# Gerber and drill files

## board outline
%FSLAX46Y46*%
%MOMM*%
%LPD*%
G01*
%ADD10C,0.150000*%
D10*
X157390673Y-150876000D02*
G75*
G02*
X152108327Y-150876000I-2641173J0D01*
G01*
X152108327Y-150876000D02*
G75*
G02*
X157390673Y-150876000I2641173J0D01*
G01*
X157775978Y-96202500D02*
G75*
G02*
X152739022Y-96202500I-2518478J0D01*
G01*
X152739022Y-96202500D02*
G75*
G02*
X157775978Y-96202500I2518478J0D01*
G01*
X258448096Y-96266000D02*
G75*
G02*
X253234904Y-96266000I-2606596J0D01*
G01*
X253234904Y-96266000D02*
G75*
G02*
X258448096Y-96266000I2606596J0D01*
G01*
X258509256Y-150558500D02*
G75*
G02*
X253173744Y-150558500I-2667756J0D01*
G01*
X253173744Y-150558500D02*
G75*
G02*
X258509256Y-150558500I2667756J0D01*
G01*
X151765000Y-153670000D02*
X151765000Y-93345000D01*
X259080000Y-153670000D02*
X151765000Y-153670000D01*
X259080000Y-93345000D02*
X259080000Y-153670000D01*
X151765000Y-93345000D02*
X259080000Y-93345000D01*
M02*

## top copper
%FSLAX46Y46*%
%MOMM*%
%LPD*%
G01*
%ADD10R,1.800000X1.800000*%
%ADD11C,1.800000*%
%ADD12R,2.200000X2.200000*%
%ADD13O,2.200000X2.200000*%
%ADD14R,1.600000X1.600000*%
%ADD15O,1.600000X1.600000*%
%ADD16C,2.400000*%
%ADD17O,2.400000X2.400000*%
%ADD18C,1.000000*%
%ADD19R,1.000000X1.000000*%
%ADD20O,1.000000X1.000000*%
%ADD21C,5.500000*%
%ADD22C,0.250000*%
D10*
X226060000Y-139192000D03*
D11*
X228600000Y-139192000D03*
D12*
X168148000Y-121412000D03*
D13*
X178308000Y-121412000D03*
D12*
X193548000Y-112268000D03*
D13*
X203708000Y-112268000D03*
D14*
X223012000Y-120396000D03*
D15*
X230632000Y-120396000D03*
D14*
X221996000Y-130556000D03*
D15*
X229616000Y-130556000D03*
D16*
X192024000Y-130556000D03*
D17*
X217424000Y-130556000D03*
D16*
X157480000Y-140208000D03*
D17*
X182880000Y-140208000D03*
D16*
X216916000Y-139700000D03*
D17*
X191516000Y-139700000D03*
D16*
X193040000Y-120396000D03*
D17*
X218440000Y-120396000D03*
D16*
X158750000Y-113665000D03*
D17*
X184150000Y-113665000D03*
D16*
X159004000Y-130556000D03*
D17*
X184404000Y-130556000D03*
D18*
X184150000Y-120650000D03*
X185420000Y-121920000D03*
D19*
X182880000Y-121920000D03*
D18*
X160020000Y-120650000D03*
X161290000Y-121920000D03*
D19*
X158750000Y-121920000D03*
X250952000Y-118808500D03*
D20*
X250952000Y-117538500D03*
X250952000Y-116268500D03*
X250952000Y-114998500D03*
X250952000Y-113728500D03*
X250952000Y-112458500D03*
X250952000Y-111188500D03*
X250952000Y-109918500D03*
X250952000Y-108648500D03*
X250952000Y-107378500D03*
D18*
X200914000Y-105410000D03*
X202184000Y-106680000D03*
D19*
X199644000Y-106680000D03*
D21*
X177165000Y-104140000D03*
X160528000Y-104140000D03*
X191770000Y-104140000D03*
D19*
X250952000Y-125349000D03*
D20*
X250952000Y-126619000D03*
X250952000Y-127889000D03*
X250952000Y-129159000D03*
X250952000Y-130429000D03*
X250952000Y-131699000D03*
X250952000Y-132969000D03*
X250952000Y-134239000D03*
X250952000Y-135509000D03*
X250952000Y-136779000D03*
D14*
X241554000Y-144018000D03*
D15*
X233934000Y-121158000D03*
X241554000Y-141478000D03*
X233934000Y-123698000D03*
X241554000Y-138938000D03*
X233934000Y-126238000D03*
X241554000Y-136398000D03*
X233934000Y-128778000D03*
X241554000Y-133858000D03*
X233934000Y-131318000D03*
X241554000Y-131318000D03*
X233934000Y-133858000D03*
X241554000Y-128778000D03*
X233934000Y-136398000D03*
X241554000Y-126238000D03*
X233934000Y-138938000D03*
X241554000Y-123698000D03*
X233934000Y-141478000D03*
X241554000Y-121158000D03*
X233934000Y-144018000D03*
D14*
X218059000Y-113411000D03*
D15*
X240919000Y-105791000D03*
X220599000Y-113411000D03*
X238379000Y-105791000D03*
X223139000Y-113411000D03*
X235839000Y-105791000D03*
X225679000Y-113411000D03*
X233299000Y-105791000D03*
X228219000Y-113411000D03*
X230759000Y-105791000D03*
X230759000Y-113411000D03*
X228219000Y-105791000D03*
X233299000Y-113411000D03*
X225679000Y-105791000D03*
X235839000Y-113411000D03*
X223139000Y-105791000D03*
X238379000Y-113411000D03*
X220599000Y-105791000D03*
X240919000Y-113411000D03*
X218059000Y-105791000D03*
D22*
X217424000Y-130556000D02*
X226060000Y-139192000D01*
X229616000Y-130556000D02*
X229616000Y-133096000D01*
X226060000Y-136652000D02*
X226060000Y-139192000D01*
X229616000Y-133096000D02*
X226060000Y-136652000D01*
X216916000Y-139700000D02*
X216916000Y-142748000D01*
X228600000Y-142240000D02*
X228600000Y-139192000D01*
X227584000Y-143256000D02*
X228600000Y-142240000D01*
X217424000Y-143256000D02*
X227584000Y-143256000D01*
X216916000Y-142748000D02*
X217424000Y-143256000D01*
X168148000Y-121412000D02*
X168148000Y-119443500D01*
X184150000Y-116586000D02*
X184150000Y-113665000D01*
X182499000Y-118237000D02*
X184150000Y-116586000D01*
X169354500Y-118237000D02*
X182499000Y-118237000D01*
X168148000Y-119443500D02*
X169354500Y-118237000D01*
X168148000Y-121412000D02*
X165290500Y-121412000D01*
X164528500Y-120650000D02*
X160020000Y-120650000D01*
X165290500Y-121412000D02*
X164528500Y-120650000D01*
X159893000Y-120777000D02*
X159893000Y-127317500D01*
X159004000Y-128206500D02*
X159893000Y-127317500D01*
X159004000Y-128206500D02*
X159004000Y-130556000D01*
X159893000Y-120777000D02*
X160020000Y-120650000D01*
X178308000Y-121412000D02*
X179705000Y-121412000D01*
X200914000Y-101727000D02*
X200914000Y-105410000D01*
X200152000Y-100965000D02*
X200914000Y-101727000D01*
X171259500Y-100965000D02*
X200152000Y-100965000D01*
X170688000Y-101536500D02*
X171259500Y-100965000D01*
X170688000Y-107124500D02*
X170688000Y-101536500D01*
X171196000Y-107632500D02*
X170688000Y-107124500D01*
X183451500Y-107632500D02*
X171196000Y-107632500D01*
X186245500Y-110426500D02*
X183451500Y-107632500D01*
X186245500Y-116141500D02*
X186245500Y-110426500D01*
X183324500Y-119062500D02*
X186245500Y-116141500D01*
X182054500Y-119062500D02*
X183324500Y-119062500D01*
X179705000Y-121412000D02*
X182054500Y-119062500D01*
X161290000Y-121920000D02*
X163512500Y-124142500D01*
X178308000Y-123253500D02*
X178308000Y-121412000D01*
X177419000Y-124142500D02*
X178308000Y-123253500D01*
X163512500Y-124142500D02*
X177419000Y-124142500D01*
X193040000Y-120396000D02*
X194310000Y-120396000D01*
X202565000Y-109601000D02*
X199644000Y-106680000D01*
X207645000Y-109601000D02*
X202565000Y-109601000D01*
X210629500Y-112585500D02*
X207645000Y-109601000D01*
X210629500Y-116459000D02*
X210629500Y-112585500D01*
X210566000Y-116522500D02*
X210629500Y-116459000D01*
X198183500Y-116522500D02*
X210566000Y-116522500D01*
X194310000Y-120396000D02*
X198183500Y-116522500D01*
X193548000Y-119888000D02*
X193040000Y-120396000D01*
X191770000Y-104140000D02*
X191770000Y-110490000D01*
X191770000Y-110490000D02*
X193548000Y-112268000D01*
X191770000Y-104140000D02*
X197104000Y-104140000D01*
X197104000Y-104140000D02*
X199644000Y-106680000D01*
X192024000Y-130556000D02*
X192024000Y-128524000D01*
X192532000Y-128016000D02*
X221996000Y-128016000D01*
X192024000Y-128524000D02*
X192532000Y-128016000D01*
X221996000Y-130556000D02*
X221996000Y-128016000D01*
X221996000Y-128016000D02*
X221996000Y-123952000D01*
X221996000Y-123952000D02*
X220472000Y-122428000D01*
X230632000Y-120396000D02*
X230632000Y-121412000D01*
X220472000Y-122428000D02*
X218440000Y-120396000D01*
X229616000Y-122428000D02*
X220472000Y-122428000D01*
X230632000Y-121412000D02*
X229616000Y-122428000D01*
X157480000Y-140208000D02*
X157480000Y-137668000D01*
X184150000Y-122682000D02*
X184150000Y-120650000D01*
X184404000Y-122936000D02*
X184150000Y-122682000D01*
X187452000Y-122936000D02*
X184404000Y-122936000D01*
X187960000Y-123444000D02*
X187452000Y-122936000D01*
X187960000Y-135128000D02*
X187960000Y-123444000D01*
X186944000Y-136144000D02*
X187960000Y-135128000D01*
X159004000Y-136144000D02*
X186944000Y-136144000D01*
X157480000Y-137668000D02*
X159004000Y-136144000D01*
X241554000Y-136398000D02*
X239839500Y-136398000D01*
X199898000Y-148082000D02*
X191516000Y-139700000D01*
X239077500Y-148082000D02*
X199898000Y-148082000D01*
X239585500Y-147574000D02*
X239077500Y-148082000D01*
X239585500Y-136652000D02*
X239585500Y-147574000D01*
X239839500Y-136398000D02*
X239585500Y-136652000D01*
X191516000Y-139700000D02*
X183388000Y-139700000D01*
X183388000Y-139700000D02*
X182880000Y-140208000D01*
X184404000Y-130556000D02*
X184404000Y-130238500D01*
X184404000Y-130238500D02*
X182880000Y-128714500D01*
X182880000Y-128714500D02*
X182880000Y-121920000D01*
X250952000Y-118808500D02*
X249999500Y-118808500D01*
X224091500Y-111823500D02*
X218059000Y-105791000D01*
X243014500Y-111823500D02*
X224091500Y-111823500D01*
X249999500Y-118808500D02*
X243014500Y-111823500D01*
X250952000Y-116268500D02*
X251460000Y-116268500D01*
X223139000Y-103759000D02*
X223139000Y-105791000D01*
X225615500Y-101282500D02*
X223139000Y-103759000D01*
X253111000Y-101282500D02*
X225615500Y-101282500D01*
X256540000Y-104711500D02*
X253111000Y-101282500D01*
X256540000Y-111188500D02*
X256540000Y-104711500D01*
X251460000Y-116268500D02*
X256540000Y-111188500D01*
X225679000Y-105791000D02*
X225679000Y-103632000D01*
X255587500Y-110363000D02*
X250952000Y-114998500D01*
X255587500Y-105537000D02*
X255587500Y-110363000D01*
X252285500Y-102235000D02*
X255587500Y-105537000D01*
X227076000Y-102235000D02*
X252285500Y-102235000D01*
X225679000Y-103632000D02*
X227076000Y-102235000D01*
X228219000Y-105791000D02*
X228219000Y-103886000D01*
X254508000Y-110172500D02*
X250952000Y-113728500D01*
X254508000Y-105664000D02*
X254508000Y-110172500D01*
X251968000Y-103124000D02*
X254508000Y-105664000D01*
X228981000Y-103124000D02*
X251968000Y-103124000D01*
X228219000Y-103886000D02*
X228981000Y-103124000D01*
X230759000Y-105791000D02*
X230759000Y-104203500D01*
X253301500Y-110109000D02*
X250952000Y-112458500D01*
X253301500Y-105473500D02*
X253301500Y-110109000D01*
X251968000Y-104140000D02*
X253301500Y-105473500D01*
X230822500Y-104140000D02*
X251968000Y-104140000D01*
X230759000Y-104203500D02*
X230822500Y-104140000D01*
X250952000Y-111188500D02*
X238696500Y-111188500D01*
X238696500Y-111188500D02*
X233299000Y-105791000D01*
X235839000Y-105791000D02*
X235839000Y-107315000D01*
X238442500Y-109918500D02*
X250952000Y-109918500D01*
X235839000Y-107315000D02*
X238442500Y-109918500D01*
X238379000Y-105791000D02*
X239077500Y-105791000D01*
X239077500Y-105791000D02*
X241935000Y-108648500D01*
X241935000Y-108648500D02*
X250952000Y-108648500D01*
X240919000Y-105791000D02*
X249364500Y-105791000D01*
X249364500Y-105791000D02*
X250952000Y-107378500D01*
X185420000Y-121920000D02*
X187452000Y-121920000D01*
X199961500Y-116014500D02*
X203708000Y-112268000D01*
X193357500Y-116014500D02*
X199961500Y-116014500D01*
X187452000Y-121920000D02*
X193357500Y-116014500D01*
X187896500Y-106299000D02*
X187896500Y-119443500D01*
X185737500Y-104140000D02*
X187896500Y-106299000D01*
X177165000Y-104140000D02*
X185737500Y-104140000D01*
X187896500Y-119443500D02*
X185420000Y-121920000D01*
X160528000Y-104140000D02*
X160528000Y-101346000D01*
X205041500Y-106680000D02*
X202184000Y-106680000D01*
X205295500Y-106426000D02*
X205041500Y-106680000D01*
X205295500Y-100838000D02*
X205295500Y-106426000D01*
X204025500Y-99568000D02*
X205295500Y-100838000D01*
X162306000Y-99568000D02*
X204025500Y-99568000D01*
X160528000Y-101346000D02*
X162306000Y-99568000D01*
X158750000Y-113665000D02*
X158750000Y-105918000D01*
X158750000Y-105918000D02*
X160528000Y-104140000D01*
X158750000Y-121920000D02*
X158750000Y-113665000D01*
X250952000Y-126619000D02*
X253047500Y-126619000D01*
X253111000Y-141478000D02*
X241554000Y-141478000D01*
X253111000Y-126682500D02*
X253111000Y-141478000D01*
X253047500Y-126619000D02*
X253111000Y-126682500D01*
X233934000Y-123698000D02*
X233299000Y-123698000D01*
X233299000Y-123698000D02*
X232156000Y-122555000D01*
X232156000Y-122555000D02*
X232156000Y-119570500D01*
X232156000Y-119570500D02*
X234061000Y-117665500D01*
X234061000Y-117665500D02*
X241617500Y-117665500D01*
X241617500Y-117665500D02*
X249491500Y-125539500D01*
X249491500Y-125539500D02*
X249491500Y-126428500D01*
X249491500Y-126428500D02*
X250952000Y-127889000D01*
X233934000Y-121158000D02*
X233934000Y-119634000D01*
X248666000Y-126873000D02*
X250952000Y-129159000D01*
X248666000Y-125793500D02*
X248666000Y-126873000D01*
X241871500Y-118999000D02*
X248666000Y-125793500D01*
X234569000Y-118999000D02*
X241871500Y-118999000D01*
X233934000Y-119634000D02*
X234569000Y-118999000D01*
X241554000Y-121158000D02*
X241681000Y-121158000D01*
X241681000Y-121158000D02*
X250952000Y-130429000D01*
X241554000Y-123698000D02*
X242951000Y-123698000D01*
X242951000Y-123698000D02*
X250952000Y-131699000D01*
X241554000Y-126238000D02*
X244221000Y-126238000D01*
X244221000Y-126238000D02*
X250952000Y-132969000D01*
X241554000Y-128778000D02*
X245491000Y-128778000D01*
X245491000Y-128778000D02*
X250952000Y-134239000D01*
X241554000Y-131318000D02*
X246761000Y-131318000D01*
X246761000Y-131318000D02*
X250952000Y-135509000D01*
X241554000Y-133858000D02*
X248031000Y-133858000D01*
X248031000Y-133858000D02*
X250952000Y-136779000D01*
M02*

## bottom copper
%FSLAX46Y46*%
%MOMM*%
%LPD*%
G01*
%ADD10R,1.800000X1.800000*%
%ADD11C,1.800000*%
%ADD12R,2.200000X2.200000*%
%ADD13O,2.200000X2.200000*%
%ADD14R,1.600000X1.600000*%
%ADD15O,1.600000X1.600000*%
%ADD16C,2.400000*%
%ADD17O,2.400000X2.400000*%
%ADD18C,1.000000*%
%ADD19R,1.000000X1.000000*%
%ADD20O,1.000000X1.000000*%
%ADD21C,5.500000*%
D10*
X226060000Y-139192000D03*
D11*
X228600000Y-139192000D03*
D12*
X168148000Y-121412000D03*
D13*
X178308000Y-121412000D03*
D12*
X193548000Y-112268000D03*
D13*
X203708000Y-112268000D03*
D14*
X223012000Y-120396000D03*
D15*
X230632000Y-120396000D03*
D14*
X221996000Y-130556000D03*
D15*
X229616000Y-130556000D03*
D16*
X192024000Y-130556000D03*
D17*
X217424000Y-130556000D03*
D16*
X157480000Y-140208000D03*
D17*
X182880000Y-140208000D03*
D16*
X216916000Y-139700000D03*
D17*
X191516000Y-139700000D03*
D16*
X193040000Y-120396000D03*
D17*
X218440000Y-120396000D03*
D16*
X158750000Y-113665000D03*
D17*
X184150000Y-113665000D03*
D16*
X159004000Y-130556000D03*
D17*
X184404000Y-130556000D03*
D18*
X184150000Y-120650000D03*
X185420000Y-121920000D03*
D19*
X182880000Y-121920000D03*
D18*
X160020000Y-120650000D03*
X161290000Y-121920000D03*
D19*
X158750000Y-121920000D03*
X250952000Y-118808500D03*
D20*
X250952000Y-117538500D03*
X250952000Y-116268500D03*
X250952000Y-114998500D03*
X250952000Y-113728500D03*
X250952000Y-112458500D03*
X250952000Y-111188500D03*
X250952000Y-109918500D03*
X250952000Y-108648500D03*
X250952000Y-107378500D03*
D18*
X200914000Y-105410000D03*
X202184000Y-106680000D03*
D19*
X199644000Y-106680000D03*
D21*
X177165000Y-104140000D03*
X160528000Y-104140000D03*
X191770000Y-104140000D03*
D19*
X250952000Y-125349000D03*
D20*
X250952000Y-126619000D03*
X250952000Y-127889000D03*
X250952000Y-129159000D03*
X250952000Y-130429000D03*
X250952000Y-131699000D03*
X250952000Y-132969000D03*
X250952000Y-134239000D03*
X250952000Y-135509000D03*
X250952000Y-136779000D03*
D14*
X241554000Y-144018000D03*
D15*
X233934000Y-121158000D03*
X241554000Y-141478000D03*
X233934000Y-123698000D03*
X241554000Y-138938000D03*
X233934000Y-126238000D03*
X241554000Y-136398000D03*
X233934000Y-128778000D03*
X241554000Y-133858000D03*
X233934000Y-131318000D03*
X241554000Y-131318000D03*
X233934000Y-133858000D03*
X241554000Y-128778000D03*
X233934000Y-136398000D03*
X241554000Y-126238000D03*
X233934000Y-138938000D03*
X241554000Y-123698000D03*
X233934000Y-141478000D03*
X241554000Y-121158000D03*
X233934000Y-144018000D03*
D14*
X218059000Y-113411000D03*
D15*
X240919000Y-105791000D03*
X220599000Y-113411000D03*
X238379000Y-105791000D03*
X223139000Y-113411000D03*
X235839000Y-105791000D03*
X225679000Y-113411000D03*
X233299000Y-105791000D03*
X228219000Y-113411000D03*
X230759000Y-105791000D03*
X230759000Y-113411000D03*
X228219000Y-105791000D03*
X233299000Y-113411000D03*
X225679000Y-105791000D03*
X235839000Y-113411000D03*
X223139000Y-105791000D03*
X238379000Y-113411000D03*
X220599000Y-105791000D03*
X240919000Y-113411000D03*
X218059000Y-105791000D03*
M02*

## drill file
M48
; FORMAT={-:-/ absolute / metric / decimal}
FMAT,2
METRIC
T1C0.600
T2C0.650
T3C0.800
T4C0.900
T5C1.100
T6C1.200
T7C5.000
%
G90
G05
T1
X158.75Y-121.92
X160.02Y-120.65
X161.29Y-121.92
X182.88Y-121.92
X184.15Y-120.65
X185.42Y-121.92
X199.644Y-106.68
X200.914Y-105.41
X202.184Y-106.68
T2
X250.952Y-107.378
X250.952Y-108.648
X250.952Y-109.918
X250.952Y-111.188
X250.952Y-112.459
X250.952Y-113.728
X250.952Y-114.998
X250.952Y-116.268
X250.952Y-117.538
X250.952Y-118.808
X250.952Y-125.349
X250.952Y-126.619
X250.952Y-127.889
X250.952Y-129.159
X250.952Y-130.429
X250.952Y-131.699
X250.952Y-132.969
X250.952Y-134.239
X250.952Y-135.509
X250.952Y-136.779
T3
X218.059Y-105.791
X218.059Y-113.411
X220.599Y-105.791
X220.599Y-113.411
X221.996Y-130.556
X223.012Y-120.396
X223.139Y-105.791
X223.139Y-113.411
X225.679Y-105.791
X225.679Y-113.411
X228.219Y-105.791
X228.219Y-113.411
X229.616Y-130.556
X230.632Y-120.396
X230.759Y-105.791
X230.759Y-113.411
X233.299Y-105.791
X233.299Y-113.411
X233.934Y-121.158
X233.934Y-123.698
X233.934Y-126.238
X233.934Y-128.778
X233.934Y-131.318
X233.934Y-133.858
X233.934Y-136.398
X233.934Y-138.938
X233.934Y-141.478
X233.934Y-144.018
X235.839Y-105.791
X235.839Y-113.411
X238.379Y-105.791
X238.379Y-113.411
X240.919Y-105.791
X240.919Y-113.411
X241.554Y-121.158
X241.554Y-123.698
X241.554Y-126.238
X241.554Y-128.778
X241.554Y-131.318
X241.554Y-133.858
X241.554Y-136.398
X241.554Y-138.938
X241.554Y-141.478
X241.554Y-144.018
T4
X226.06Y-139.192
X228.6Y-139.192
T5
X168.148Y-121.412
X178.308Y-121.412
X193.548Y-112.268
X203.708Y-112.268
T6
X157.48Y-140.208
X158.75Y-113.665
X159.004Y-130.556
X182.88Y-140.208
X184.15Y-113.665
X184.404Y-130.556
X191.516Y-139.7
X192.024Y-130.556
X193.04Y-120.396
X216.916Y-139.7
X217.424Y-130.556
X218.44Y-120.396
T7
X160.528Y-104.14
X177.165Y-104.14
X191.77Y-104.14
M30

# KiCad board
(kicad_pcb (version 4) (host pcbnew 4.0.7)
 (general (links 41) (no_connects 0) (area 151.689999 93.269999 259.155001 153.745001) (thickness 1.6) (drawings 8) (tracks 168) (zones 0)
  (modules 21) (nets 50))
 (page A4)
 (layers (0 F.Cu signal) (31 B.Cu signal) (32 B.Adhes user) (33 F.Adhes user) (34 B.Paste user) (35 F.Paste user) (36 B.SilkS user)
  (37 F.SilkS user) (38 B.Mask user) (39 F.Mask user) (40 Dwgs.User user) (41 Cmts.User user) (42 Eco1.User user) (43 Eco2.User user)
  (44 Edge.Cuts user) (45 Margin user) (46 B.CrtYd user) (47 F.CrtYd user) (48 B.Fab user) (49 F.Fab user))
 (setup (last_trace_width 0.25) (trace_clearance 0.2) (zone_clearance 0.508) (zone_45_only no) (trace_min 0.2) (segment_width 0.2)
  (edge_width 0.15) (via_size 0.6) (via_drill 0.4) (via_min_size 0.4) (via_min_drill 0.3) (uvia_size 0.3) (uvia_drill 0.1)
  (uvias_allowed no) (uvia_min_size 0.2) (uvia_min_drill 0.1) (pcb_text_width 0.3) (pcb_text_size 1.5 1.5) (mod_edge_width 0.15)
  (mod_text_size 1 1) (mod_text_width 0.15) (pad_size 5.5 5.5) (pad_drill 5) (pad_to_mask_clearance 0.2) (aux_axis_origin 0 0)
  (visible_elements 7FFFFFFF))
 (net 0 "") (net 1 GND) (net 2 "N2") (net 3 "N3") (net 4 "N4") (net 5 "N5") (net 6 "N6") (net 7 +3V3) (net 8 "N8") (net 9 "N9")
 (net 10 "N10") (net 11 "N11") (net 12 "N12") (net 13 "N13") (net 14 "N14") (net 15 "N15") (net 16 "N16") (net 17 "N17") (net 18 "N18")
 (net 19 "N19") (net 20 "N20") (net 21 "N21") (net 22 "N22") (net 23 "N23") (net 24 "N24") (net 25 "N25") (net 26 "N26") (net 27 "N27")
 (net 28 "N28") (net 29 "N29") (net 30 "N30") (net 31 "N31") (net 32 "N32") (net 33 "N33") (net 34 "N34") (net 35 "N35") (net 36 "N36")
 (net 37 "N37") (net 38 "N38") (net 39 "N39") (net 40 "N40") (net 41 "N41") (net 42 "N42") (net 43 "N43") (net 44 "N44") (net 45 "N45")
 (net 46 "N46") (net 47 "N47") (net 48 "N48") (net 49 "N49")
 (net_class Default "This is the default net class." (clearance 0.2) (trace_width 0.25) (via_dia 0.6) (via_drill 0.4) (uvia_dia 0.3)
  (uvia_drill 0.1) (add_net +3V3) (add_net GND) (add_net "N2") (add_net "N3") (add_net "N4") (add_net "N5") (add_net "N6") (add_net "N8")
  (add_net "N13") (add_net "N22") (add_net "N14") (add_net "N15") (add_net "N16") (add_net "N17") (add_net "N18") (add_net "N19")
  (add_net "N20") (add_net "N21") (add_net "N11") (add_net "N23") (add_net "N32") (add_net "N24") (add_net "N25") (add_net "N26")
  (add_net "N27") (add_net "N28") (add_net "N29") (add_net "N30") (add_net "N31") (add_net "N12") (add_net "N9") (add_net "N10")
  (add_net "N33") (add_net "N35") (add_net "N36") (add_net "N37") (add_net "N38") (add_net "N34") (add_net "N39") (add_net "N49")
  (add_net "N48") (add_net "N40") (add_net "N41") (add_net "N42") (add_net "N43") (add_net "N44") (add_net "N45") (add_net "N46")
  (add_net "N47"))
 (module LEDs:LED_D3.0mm (layer F.Cu) (at 226.06 139.192)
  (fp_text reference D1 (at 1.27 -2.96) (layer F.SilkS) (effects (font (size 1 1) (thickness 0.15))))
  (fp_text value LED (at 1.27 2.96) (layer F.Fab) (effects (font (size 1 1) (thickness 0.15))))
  (pad 1 thru_hole rect (at 0 0) (size 1.8 1.8) (drill 0.9) (layers *.Cu *.Mask) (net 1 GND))
  (pad 2 thru_hole circle (at 2.54 0) (size 1.8 1.8) (drill 0.9) (layers *.Cu *.Mask) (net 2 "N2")))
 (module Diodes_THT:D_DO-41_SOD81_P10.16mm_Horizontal (layer F.Cu) (at 168.148 121.412)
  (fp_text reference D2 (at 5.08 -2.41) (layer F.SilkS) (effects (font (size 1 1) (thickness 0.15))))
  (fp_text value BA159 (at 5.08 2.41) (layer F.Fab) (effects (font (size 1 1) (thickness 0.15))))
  (pad 1 thru_hole rect (at 0 0) (size 2.2 2.2) (drill 1.1) (layers *.Cu *.Mask) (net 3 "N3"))
  (pad 2 thru_hole oval (at 10.16 0) (size 2.2 2.2) (drill 1.1) (layers *.Cu *.Mask) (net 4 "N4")))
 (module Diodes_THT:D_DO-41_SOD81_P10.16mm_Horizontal (layer F.Cu) (at 193.548 112.268)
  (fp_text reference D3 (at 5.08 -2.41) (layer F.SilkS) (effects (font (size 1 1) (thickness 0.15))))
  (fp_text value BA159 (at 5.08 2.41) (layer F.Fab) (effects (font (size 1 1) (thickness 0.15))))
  (pad 1 thru_hole rect (at 0 0) (size 2.2 2.2) (drill 1.1) (layers *.Cu *.Mask) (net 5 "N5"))
  (pad 2 thru_hole oval (at 10.16 0) (size 2.2 2.2) (drill 1.1) (layers *.Cu *.Mask) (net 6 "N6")))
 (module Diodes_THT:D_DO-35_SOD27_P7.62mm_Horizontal (layer F.Cu) (at 223.012 120.396)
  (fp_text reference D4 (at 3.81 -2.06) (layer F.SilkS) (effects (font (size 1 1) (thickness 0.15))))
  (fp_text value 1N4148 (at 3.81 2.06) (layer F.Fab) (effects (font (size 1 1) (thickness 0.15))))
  (pad 1 thru_hole rect (at 0 0) (size 1.6 1.6) (drill 0.8) (layers *.Cu *.Mask) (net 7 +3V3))
  (pad 2 thru_hole oval (at 7.62 0) (size 1.6 1.6) (drill 0.8) (layers *.Cu *.Mask) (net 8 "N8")))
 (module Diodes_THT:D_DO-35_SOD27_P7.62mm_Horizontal (layer F.Cu) (at 221.996 130.556)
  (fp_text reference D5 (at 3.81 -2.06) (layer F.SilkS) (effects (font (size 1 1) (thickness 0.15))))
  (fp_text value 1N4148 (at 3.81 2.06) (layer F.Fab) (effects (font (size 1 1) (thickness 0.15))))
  (pad 1 thru_hole rect (at 0 0) (size 1.6 1.6) (drill 0.8) (layers *.Cu *.Mask) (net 8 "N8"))
  (pad 2 thru_hole oval (at 7.62 0) (size 1.6 1.6) (drill 0.8) (layers *.Cu *.Mask) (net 1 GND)))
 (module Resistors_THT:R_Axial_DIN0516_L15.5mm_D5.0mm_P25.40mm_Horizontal (layer F.Cu) (at 192.024 130.556)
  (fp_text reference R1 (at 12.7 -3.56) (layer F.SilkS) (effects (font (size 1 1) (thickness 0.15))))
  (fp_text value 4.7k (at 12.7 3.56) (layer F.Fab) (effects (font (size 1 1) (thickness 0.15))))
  (pad 1 thru_hole circle (at 0 0) (size 2.4 2.4) (drill 1.2) (layers *.Cu *.Mask) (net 8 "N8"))
  (pad 2 thru_hole oval (at 25.4 0) (size 2.4 2.4) (drill 1.2) (layers *.Cu *.Mask) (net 1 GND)))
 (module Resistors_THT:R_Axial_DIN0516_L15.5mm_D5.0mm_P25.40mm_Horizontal (layer F.Cu) (at 157.48 140.208)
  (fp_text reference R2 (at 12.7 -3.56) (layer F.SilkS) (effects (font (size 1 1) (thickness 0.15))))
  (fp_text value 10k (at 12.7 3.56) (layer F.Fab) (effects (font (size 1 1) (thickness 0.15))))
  (pad 1 thru_hole circle (at 0 0) (size 2.4 2.4) (drill 1.2) (layers *.Cu *.Mask) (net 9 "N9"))
  (pad 2 thru_hole oval (at 25.4 0) (size 2.4 2.4) (drill 1.2) (layers *.Cu *.Mask) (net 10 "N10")))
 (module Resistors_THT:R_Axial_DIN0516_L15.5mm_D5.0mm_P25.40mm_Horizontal (layer F.Cu) (at 216.916 139.7 180)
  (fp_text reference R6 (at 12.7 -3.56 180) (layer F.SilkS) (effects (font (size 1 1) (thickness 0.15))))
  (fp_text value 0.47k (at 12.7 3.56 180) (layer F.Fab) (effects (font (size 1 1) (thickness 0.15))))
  (pad 1 thru_hole circle (at 0 0 180) (size 2.4 2.4) (drill 1.2) (layers *.Cu *.Mask) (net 2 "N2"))
  (pad 2 thru_hole oval (at 25.4 0 180) (size 2.4 2.4) (drill 1.2) (layers *.Cu *.Mask) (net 10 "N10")))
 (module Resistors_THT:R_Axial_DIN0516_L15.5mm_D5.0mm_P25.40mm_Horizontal (layer F.Cu) (at 193.04 120.396)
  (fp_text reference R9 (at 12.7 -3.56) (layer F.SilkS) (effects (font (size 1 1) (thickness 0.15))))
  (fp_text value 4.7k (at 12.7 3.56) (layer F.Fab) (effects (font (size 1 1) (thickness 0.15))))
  (pad 1 thru_hole circle (at 0 0) (size 2.4 2.4) (drill 1.2) (layers *.Cu *.Mask) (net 5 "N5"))
  (pad 2 thru_hole oval (at 25.4 0) (size 2.4 2.4) (drill 1.2) (layers *.Cu *.Mask) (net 8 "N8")))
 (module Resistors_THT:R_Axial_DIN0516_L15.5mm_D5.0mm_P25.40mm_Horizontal (layer F.Cu) (at 158.75 113.665)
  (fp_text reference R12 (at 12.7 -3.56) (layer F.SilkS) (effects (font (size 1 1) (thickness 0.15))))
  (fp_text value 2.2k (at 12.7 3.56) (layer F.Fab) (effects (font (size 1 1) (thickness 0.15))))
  (pad 1 thru_hole circle (at 0 0) (size 2.4 2.4) (drill 1.2) (layers *.Cu *.Mask) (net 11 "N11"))
  (pad 2 thru_hole oval (at 25.4 0) (size 2.4 2.4) (drill 1.2) (layers *.Cu *.Mask) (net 3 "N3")))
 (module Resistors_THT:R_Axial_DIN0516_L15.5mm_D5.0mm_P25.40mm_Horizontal (layer F.Cu) (at 159.004 130.556)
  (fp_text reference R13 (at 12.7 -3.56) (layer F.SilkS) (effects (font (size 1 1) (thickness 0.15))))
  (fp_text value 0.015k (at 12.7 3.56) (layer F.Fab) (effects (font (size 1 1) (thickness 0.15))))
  (pad 1 thru_hole circle (at 0 0) (size 2.4 2.4) (drill 1.2) (layers *.Cu *.Mask) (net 3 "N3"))
  (pad 2 thru_hole oval (at 25.4 0) (size 2.4 2.4) (drill 1.2) (layers *.Cu *.Mask) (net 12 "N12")))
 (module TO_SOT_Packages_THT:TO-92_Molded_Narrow (layer F.Cu) (at 182.88 121.92)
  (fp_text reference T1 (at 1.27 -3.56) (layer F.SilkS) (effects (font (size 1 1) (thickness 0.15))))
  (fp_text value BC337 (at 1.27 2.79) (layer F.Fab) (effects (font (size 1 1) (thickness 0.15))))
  (pad 2 thru_hole circle (at 1.27 -1.27 90) (size 1 1) (drill 0.6) (layers *.Cu *.Mask) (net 9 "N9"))
  (pad 3 thru_hole circle (at 2.54 0 90) (size 1 1) (drill 0.6) (layers *.Cu *.Mask) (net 6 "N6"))
  (pad 1 thru_hole rect (at 0 0 90) (size 1 1) (drill 0.6) (layers *.Cu *.Mask) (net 12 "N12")))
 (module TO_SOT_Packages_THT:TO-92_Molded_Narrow (layer F.Cu) (at 158.75 121.92)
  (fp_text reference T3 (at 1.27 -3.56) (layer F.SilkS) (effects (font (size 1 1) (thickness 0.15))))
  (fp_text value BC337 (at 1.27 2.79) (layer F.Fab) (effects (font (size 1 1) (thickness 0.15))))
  (pad 2 thru_hole circle (at 1.27 -1.27 90) (size 1 1) (drill 0.6) (layers *.Cu *.Mask) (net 3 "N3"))
  (pad 3 thru_hole circle (at 2.54 0 90) (size 1 1) (drill 0.6) (layers *.Cu *.Mask) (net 4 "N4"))
  (pad 1 thru_hole rect (at 0 0 90) (size 1 1) (drill 0.6) (layers *.Cu *.Mask) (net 11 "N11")))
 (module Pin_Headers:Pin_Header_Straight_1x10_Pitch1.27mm (layer F.Cu) (at 250.952 118.8085 180)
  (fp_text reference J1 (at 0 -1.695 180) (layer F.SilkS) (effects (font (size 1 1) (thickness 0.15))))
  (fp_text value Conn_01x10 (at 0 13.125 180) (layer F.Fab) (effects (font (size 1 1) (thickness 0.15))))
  (pad 1 thru_hole rect (at 0 0 180) (size 1 1) (drill 0.65) (layers *.Cu *.Mask) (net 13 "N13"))
  (pad 2 thru_hole oval (at 0 1.27 180) (size 1 1) (drill 0.65) (layers *.Cu *.Mask) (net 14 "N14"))
  (pad 3 thru_hole oval (at 0 2.54 180) (size 1 1) (drill 0.65) (layers *.Cu *.Mask) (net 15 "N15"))
  (pad 4 thru_hole oval (at 0 3.81 180) (size 1 1) (drill 0.65) (layers *.Cu *.Mask) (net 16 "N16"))
  (pad 5 thru_hole oval (at 0 5.08 180) (size 1 1) (drill 0.65) (layers *.Cu *.Mask) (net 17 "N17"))
  (pad 6 thru_hole oval (at 0 6.35 180) (size 1 1) (drill 0.65) (layers *.Cu *.Mask) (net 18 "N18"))
  (pad 7 thru_hole oval (at 0 7.62 180) (size 1 1) (drill 0.65) (layers *.Cu *.Mask) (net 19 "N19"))
  (pad 8 thru_hole oval (at 0 8.89 180) (size 1 1) (drill 0.65) (layers *.Cu *.Mask) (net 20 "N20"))
  (pad 9 thru_hole oval (at 0 10.16 180) (size 1 1) (drill 0.65) (layers *.Cu *.Mask) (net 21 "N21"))
  (pad 10 thru_hole oval (at 0 11.43 180) (size 1 1) (drill 0.65) (layers *.Cu *.Mask) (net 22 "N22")))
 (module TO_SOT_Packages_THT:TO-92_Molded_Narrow (layer F.Cu) (at 199.644 106.68)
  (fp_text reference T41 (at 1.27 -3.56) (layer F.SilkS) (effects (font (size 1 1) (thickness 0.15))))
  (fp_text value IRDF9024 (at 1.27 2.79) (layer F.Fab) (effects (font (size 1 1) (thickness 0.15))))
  (pad 2 thru_hole circle (at 1.27 -1.27 90) (size 1 1) (drill 0.6) (layers *.Cu *.Mask) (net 4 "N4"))
  (pad 3 thru_hole circle (at 2.54 0 90) (size 1 1) (drill 0.6) (layers *.Cu *.Mask) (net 11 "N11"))
  (pad 1 thru_hole rect (at 0 0 90) (size 1 1) (drill 0.6) (layers *.Cu *.Mask) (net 5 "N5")))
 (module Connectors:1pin (layer F.Cu) (at 177.165 104.14)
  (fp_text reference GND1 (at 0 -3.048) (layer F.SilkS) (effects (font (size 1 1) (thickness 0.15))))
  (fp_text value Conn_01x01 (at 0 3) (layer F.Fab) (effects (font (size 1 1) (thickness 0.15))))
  (pad 1 thru_hole circle (at 0 0) (size 5.5 5.5) (drill 5) (layers *.Cu *.Mask) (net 6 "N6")))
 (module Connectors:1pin (layer F.Cu) (at 160.528 104.14)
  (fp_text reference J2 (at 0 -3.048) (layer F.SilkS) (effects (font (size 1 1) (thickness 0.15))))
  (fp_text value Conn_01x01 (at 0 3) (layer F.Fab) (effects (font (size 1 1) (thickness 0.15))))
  (pad 1 thru_hole circle (at 0 0) (size 5.5 5.5) (drill 5) (layers *.Cu *.Mask) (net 11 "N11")))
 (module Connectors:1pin (layer F.Cu) (at 191.77 104.14)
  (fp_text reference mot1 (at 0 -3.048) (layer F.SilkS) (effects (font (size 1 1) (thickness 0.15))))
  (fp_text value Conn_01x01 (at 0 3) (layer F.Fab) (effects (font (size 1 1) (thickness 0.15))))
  (pad 1 thru_hole circle (at 0 0) (size 5.5 5.5) (drill 5) (layers *.Cu *.Mask) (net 5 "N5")))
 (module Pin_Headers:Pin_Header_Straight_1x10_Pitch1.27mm (layer F.Cu) (at 250.952 125.349)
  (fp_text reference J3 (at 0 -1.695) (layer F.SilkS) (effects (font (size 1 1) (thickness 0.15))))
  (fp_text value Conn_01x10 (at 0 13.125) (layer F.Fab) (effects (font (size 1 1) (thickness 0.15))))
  (pad 1 thru_hole rect (at 0 0) (size 1 1) (drill 0.65) (layers *.Cu *.Mask) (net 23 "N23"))
  (pad 2 thru_hole oval (at 0 1.27) (size 1 1) (drill 0.65) (layers *.Cu *.Mask) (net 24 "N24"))
  (pad 3 thru_hole oval (at 0 2.54) (size 1 1) (drill 0.65) (layers *.Cu *.Mask) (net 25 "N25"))
  (pad 4 thru_hole oval (at 0 3.81) (size 1 1) (drill 0.65) (layers *.Cu *.Mask) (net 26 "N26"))
  (pad 5 thru_hole oval (at 0 5.08) (size 1 1) (drill 0.65) (layers *.Cu *.Mask) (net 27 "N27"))
  (pad 6 thru_hole oval (at 0 6.35) (size 1 1) (drill 0.65) (layers *.Cu *.Mask) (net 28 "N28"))
  (pad 7 thru_hole oval (at 0 7.62) (size 1 1) (drill 0.65) (layers *.Cu *.Mask) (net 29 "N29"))
  (pad 8 thru_hole oval (at 0 8.89) (size 1 1) (drill 0.65) (layers *.Cu *.Mask) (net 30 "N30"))
  (pad 9 thru_hole oval (at 0 10.16) (size 1 1) (drill 0.65) (layers *.Cu *.Mask) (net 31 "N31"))
  (pad 10 thru_hole oval (at 0 11.43) (size 1 1) (drill 0.65) (layers *.Cu *.Mask) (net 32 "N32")))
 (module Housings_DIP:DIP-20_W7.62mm (layer F.Cu) (at 241.554 144.018 180)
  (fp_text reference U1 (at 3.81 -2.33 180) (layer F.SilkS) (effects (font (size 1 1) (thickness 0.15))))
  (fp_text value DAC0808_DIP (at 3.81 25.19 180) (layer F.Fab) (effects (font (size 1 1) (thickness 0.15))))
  (pad 1 thru_hole rect (at 0 0 180) (size 1.6 1.6) (drill 0.8) (layers *.Cu *.Mask) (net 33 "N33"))
  (pad 11 thru_hole oval (at 7.62 22.86 180) (size 1.6 1.6) (drill 0.8) (layers *.Cu *.Mask) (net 26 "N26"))
  (pad 2 thru_hole oval (at 0 2.54 180) (size 1.6 1.6) (drill 0.8) (layers *.Cu *.Mask) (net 24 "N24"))
  (pad 12 thru_hole oval (at 7.62 20.32 180) (size 1.6 1.6) (drill 0.8) (layers *.Cu *.Mask) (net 25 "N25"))
  (pad 3 thru_hole oval (at 0 5.08 180) (size 1.6 1.6) (drill 0.8) (layers *.Cu *.Mask) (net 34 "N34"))
  (pad 13 thru_hole oval (at 7.62 17.78 180) (size 1.6 1.6) (drill 0.8) (layers *.Cu *.Mask) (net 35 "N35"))
  (pad 4 thru_hole oval (at 0 7.62 180) (size 1.6 1.6) (drill 0.8) (layers *.Cu *.Mask) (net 10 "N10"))
  (pad 14 thru_hole oval (at 7.62 15.24 180) (size 1.6 1.6) (drill 0.8) (layers *.Cu *.Mask) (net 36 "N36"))
  (pad 5 thru_hole oval (at 0 10.16 180) (size 1.6 1.6) (drill 0.8) (layers *.Cu *.Mask) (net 32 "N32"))
  (pad 15 thru_hole oval (at 7.62 12.7 180) (size 1.6 1.6) (drill 0.8) (layers *.Cu *.Mask) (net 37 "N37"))
  (pad 6 thru_hole oval (at 0 12.7 180) (size 1.6 1.6) (drill 0.8) (layers *.Cu *.Mask) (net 31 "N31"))
  (pad 16 thru_hole oval (at 7.62 10.16 180) (size 1.6 1.6) (drill 0.8) (layers *.Cu *.Mask) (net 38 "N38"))
  (pad 7 thru_hole oval (at 0 15.24 180) (size 1.6 1.6) (drill 0.8) (layers *.Cu *.Mask) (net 30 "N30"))
  (pad 17 thru_hole oval (at 7.62 7.62 180) (size 1.6 1.6) (drill 0.8) (layers *.Cu *.Mask))
  (pad 8 thru_hole oval (at 0 17.78 180) (size 1.6 1.6) (drill 0.8) (layers *.Cu *.Mask) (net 29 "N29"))
  (pad 18 thru_hole oval (at 7.62 5.08 180) (size 1.6 1.6) (drill 0.8) (layers *.Cu *.Mask))
  (pad 9 thru_hole oval (at 0 20.32 180) (size 1.6 1.6) (drill 0.8) (layers *.Cu *.Mask) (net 28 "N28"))
  (pad 19 thru_hole oval (at 7.62 2.54 180) (size 1.6 1.6) (drill 0.8) (layers *.Cu *.Mask))
  (pad 10 thru_hole oval (at 0 22.86 180) (size 1.6 1.6) (drill 0.8) (layers *.Cu *.Mask) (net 27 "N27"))
  (pad 20 thru_hole oval (at 7.62 0 180) (size 1.6 1.6) (drill 0.8) (layers *.Cu *.Mask)))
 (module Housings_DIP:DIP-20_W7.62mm (layer F.Cu) (at 218.059 113.411 90)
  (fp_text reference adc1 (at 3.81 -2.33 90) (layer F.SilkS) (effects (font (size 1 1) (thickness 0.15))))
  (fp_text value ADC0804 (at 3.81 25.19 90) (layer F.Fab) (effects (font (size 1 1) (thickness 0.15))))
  (pad 1 thru_hole rect (at 0 0 90) (size 1.6 1.6) (drill 0.8) (layers *.Cu *.Mask) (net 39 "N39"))
  (pad 11 thru_hole oval (at 7.62 22.86 90) (size 1.6 1.6) (drill 0.8) (layers *.Cu *.Mask) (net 22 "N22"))
  (pad 2 thru_hole oval (at 0 2.54 90) (size 1.6 1.6) (drill 0.8) (layers *.Cu *.Mask) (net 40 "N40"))
  (pad 12 thru_hole oval (at 7.62 20.32 90) (size 1.6 1.6) (drill 0.8) (layers *.Cu *.Mask) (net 21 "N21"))
  (pad 3 thru_hole oval (at 0 5.08 90) (size 1.6 1.6) (drill 0.8) (layers *.Cu *.Mask) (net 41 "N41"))
  (pad 13 thru_hole oval (at 7.62 17.78 90) (size 1.6 1.6) (drill 0.8) (layers *.Cu *.Mask) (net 20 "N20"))
  (pad 4 thru_hole oval (at 0 7.62 90) (size 1.6 1.6) (drill 0.8) (layers *.Cu *.Mask) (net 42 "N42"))
  (pad 14 thru_hole oval (at 7.62 15.24 90) (size 1.6 1.6) (drill 0.8) (layers *.Cu *.Mask) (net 19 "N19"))
  (pad 5 thru_hole oval (at 0 10.16 90) (size 1.6 1.6) (drill 0.8) (layers *.Cu *.Mask) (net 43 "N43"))
  (pad 15 thru_hole oval (at 7.62 12.7 90) (size 1.6 1.6) (drill 0.8) (layers *.Cu *.Mask) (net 18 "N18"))
  (pad 6 thru_hole oval (at 0 12.7 90) (size 1.6 1.6) (drill 0.8) (layers *.Cu *.Mask) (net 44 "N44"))
  (pad 16 thru_hole oval (at 7.62 10.16 90) (size 1.6 1.6) (drill 0.8) (layers *.Cu *.Mask) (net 17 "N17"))
  (pad 7 thru_hole oval (at 0 15.24 90) (size 1.6 1.6) (drill 0.8) (layers *.Cu *.Mask) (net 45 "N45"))
  (pad 17 thru_hole oval (at 7.62 7.62 90) (size 1.6 1.6) (drill 0.8) (layers *.Cu *.Mask) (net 16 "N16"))
  (pad 8 thru_hole oval (at 0 17.78 90) (size 1.6 1.6) (drill 0.8) (layers *.Cu *.Mask) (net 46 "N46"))
  (pad 18 thru_hole oval (at 7.62 5.08 90) (size 1.6 1.6) (drill 0.8) (layers *.Cu *.Mask) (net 15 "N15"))
  (pad 9 thru_hole oval (at 0 20.32 90) (size 1.6 1.6) (drill 0.8) (layers *.Cu *.Mask) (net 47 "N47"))
  (pad 19 thru_hole oval (at 7.62 2.54 90) (size 1.6 1.6) (drill 0.8) (layers *.Cu *.Mask) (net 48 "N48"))
  (pad 10 thru_hole oval (at 0 22.86 90) (size 1.6 1.6) (drill 0.8) (layers *.Cu *.Mask) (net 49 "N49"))
  (pad 20 thru_hole oval (at 7.62 0 90) (size 1.6 1.6) (drill 0.8) (layers *.Cu *.Mask) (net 13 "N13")))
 (gr_circle (center 154.7495 150.876) (end 157.099 152.0825) (layer Edge.Cuts) (width 0.15))
 (gr_circle (center 155.2575 96.2025) (end 157.353 97.5995) (layer Edge.Cuts) (width 0.15))
 (gr_circle (center 255.8415 96.266) (end 255.9685 98.8695) (layer Edge.Cuts) (width 0.15))
 (gr_circle (center 255.8415 150.5585) (end 257.4925 152.654) (layer Edge.Cuts) (width 0.15))
 (gr_line (start 151.765 153.67) (end 151.765 93.345) (angle 90) (layer Edge.Cuts) (width 0.15))
 (gr_line (start 259.08 153.67) (end 151.765 153.67) (angle 90) (layer Edge.Cuts) (width 0.15))
 (gr_line (start 259.08 93.345) (end 259.08 153.67) (angle 90) (layer Edge.Cuts) (width 0.15))
 (gr_line (start 151.765 93.345) (end 259.08 93.345) (angle 90) (layer Edge.Cuts) (width 0.15))
 (segment (start 217.424 130.556) (end 226.06 139.192) (width 0.25) (layer F.Cu) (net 1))
 (segment (start 229.616 130.556) (end 229.616 133.096) (width 0.25) (layer F.Cu) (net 1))
 (segment (start 226.06 136.652) (end 226.06 139.192) (width 0.25) (layer F.Cu) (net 1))
 (segment (start 229.616 133.096) (end 226.06 136.652) (width 0.25) (layer F.Cu) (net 1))
 (segment (start 216.916 139.7) (end 216.916 142.748) (width 0.25) (layer F.Cu) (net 2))
 (segment (start 228.6 142.24) (end 228.6 139.192) (width 0.25) (layer F.Cu) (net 2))
 (segment (start 227.584 143.256) (end 228.6 142.24) (width 0.25) (layer F.Cu) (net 2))
 (segment (start 217.424 143.256) (end 227.584 143.256) (width 0.25) (layer F.Cu) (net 2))
 (segment (start 216.916 142.748) (end 217.424 143.256) (width 0.25) (layer F.Cu) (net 2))
 (segment (start 168.148 121.412) (end 168.148 119.4435) (width 0.25) (layer F.Cu) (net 3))
 (segment (start 184.15 116.586) (end 184.15 113.665) (width 0.25) (layer F.Cu) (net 3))
 (segment (start 182.499 118.237) (end 184.15 116.586) (width 0.25) (layer F.Cu) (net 3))
 (segment (start 169.3545 118.237) (end 182.499 118.237) (width 0.25) (layer F.Cu) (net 3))
 (segment (start 168.148 119.4435) (end 169.3545 118.237) (width 0.25) (layer F.Cu) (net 3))
 (segment (start 168.148 121.412) (end 165.2905 121.412) (width 0.25) (layer F.Cu) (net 3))
 (segment (start 164.5285 120.65) (end 160.02 120.65) (width 0.25) (layer F.Cu) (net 3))
 (segment (start 165.2905 121.412) (end 164.5285 120.65) (width 0.25) (layer F.Cu) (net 3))
 (segment (start 159.893 120.777) (end 159.893 127.3175) (width 0.25) (layer F.Cu) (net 3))
 (segment (start 159.004 128.2065) (end 159.893 127.3175) (width 0.25) (layer F.Cu) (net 3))
 (segment (start 159.004 128.2065) (end 159.004 130.556) (width 0.25) (layer F.Cu) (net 3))
 (segment (start 159.893 120.777) (end 160.02 120.65) (width 0.25) (layer F.Cu) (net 3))
 (segment (start 178.308 121.412) (end 179.705 121.412) (width 0.25) (layer F.Cu) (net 4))
 (segment (start 200.914 101.727) (end 200.914 105.41) (width 0.25) (layer F.Cu) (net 4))
 (segment (start 200.152 100.965) (end 200.914 101.727) (width 0.25) (layer F.Cu) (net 4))
 (segment (start 171.2595 100.965) (end 200.152 100.965) (width 0.25) (layer F.Cu) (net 4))
 (segment (start 170.688 101.5365) (end 171.2595 100.965) (width 0.25) (layer F.Cu) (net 4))
 (segment (start 170.688 107.1245) (end 170.688 101.5365) (width 0.25) (layer F.Cu) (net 4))
 (segment (start 171.196 107.6325) (end 170.688 107.1245) (width 0.25) (layer F.Cu) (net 4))
 (segment (start 183.4515 107.6325) (end 171.196 107.6325) (width 0.25) (layer F.Cu) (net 4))
 (segment (start 186.2455 110.4265) (end 183.4515 107.6325) (width 0.25) (layer F.Cu) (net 4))
 (segment (start 186.2455 116.1415) (end 186.2455 110.4265) (width 0.25) (layer F.Cu) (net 4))
 (segment (start 183.3245 119.0625) (end 186.2455 116.1415) (width 0.25) (layer F.Cu) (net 4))
 (segment (start 182.0545 119.0625) (end 183.3245 119.0625) (width 0.25) (layer F.Cu) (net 4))
 (segment (start 179.705 121.412) (end 182.0545 119.0625) (width 0.25) (layer F.Cu) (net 4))
 (segment (start 161.29 121.92) (end 163.5125 124.1425) (width 0.25) (layer F.Cu) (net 4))
 (segment (start 178.308 123.2535) (end 178.308 121.412) (width 0.25) (layer F.Cu) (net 4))
 (segment (start 177.419 124.1425) (end 178.308 123.2535) (width 0.25) (layer F.Cu) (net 4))
 (segment (start 163.5125 124.1425) (end 177.419 124.1425) (width 0.25) (layer F.Cu) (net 4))
 (segment (start 193.04 120.396) (end 194.31 120.396) (width 0.25) (layer F.Cu) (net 5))
 (segment (start 202.565 109.601) (end 199.644 106.68) (width 0.25) (layer F.Cu) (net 5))
 (segment (start 207.645 109.601) (end 202.565 109.601) (width 0.25) (layer F.Cu) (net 5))
 (segment (start 210.6295 112.5855) (end 207.645 109.601) (width 0.25) (layer F.Cu) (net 5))
 (segment (start 210.6295 116.459) (end 210.6295 112.5855) (width 0.25) (layer F.Cu) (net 5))
 (segment (start 210.566 116.5225) (end 210.6295 116.459) (width 0.25) (layer F.Cu) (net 5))
 (segment (start 198.1835 116.5225) (end 210.566 116.5225) (width 0.25) (layer F.Cu) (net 5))
 (segment (start 194.31 120.396) (end 198.1835 116.5225) (width 0.25) (layer F.Cu) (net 5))
 (segment (start 193.548 119.888) (end 193.04 120.396) (width 0.25) (layer F.Cu) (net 5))
 (segment (start 191.77 104.14) (end 191.77 110.49) (width 0.25) (layer F.Cu) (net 5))
 (segment (start 191.77 110.49) (end 193.548 112.268) (width 0.25) (layer F.Cu) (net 5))
 (segment (start 191.77 104.14) (end 197.104 104.14) (width 0.25) (layer F.Cu) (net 5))
 (segment (start 197.104 104.14) (end 199.644 106.68) (width 0.25) (layer F.Cu) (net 5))
 (segment (start 192.024 130.556) (end 192.024 128.524) (width 0.25) (layer F.Cu) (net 8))
 (segment (start 192.532 128.016) (end 221.996 128.016) (width 0.25) (layer F.Cu) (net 8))
 (segment (start 192.024 128.524) (end 192.532 128.016) (width 0.25) (layer F.Cu) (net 8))
 (segment (start 221.996 130.556) (end 221.996 128.016) (width 0.25) (layer F.Cu) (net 8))
 (segment (start 221.996 128.016) (end 221.996 123.952) (width 0.25) (layer F.Cu) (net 8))
 (segment (start 221.996 123.952) (end 220.472 122.428) (width 0.25) (layer F.Cu) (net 8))
 (segment (start 230.632 120.396) (end 230.632 121.412) (width 0.25) (layer F.Cu) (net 8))
 (segment (start 220.472 122.428) (end 218.44 120.396) (width 0.25) (layer F.Cu) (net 8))
 (segment (start 229.616 122.428) (end 220.472 122.428) (width 0.25) (layer F.Cu) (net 8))
 (segment (start 230.632 121.412) (end 229.616 122.428) (width 0.25) (layer F.Cu) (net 8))
 (segment (start 157.48 140.208) (end 157.48 137.668) (width 0.25) (layer F.Cu) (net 9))
 (segment (start 184.15 122.682) (end 184.15 120.65) (width 0.25) (layer F.Cu) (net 9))
 (segment (start 184.404 122.936) (end 184.15 122.682) (width 0.25) (layer F.Cu) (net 9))
 (segment (start 187.452 122.936) (end 184.404 122.936) (width 0.25) (layer F.Cu) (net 9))
 (segment (start 187.96 123.444) (end 187.452 122.936) (width 0.25) (layer F.Cu) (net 9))
 (segment (start 187.96 135.128) (end 187.96 123.444) (width 0.25) (layer F.Cu) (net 9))
 (segment (start 186.944 136.144) (end 187.96 135.128) (width 0.25) (layer F.Cu) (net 9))
 (segment (start 159.004 136.144) (end 186.944 136.144) (width 0.25) (layer F.Cu) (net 9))
 (segment (start 157.48 137.668) (end 159.004 136.144) (width 0.25) (layer F.Cu) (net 9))
 (segment (start 241.554 136.398) (end 239.8395 136.398) (width 0.25) (layer F.Cu) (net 10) (status 400000))
 (segment (start 199.898 148.082) (end 191.516 139.7) (width 0.25) (layer F.Cu) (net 10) (status 800000))
 (segment (start 239.0775 148.082) (end 199.898 148.082) (width 0.25) (layer F.Cu) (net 10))
 (segment (start 239.5855 147.574) (end 239.0775 148.082) (width 0.25) (layer F.Cu) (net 10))
 (segment (start 239.5855 136.652) (end 239.5855 147.574) (width 0.25) (layer F.Cu) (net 10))
 (segment (start 239.8395 136.398) (end 239.5855 136.652) (width 0.25) (layer F.Cu) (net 10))
 (segment (start 191.516 139.7) (end 183.388 139.7) (width 0.25) (layer F.Cu) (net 10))
 (segment (start 183.388 139.7) (end 182.88 140.208) (width 0.25) (layer F.Cu) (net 10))
 (segment (start 184.404 130.556) (end 184.404 130.2385) (width 0.25) (layer F.Cu) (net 12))
 (segment (start 184.404 130.2385) (end 182.88 128.7145) (width 0.25) (layer F.Cu) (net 12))
 (segment (start 182.88 128.7145) (end 182.88 121.92) (width 0.25) (layer F.Cu) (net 12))
 (segment (start 250.952 118.8085) (end 249.9995 118.8085) (width 0.25) (layer F.Cu) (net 13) (status 400000))
 (segment (start 224.0915 111.8235) (end 218.059 105.791) (width 0.25) (layer F.Cu) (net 13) (status 800000))
 (segment (start 243.0145 111.8235) (end 224.0915 111.8235) (width 0.25) (layer F.Cu) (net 13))
 (segment (start 249.9995 118.8085) (end 243.0145 111.8235) (width 0.25) (layer F.Cu) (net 13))
 (segment (start 250.952 116.2685) (end 251.46 116.2685) (width 0.25) (layer F.Cu) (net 15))
 (segment (start 223.139 103.759) (end 223.139 105.791) (width 0.25) (layer F.Cu) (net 15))
 (segment (start 225.6155 101.2825) (end 223.139 103.759) (width 0.25) (layer F.Cu) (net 15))
 (segment (start 253.111 101.2825) (end 225.6155 101.2825) (width 0.25) (layer F.Cu) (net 15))
 (segment (start 256.54 104.7115) (end 253.111 101.2825) (width 0.25) (layer F.Cu) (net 15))
 (segment (start 256.54 111.1885) (end 256.54 104.7115) (width 0.25) (layer F.Cu) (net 15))
 (segment (start 251.46 116.2685) (end 256.54 111.1885) (width 0.25) (layer F.Cu) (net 15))
 (segment (start 225.679 105.791) (end 225.679 103.632) (width 0.25) (layer F.Cu) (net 16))
 (segment (start 255.5875 110.363) (end 250.952 114.9985) (width 0.25) (layer F.Cu) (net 16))
 (segment (start 255.5875 105.537) (end 255.5875 110.363) (width 0.25) (layer F.Cu) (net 16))
 (segment (start 252.2855 102.235) (end 255.5875 105.537) (width 0.25) (layer F.Cu) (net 16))
 (segment (start 227.076 102.235) (end 252.2855 102.235) (width 0.25) (layer F.Cu) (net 16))
 (segment (start 225.679 103.632) (end 227.076 102.235) (width 0.25) (layer F.Cu) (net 16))
 (segment (start 228.219 105.791) (end 228.219 103.886) (width 0.25) (layer F.Cu) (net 17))
 (segment (start 254.508 110.1725) (end 250.952 113.7285) (width 0.25) (layer F.Cu) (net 17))
 (segment (start 254.508 105.664) (end 254.508 110.1725) (width 0.25) (layer F.Cu) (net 17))
 (segment (start 251.968 103.124) (end 254.508 105.664) (width 0.25) (layer F.Cu) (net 17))
 (segment (start 228.981 103.124) (end 251.968 103.124) (width 0.25) (layer F.Cu) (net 17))
 (segment (start 228.219 103.886) (end 228.981 103.124) (width 0.25) (layer F.Cu) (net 17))
 (segment (start 230.759 105.791) (end 230.759 104.2035) (width 0.25) (layer F.Cu) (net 18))
 (segment (start 253.3015 110.109) (end 250.952 112.4585) (width 0.25) (layer F.Cu) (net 18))
 (segment (start 253.3015 105.4735) (end 253.3015 110.109) (width 0.25) (layer F.Cu) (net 18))
 (segment (start 251.968 104.14) (end 253.3015 105.4735) (width 0.25) (layer F.Cu) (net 18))
 (segment (start 230.8225 104.14) (end 251.968 104.14) (width 0.25) (layer F.Cu) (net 18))
 (segment (start 230.759 104.2035) (end 230.8225 104.14) (width 0.25) (layer F.Cu) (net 18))
 (segment (start 250.952 111.1885) (end 238.6965 111.1885) (width 0.25) (layer F.Cu) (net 19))
 (segment (start 238.6965 111.1885) (end 233.299 105.791) (width 0.25) (layer F.Cu) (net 19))
 (segment (start 235.839 105.791) (end 235.839 107.315) (width 0.25) (layer F.Cu) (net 20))
 (segment (start 238.4425 109.9185) (end 250.952 109.9185) (width 0.25) (layer F.Cu) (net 20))
 (segment (start 235.839 107.315) (end 238.4425 109.9185) (width 0.25) (layer F.Cu) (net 20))
 (segment (start 238.379 105.791) (end 239.0775 105.791) (width 0.25) (layer F.Cu) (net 21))
 (segment (start 239.0775 105.791) (end 241.935 108.6485) (width 0.25) (layer F.Cu) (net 21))
 (segment (start 241.935 108.6485) (end 250.952 108.6485) (width 0.25) (layer F.Cu) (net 21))
 (segment (start 240.919 105.791) (end 249.3645 105.791) (width 0.25) (layer F.Cu) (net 22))
 (segment (start 249.3645 105.791) (end 250.952 107.3785) (width 0.25) (layer F.Cu) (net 22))
 (segment (start 185.42 121.92) (end 187.452 121.92) (width 0.25) (layer F.Cu) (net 6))
 (segment (start 199.9615 116.0145) (end 203.708 112.268) (width 0.25) (layer F.Cu) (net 6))
 (segment (start 193.3575 116.0145) (end 199.9615 116.0145) (width 0.25) (layer F.Cu) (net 6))
 (segment (start 187.452 121.92) (end 193.3575 116.0145) (width 0.25) (layer F.Cu) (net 6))
 (segment (start 187.8965 106.299) (end 187.8965 119.4435) (width 0.25) (layer F.Cu) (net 6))
 (segment (start 185.7375 104.14) (end 187.8965 106.299) (width 0.25) (layer F.Cu) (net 6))
 (segment (start 177.165 104.14) (end 185.7375 104.14) (width 0.25) (layer F.Cu) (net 6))
 (segment (start 187.8965 119.4435) (end 185.42 121.92) (width 0.25) (layer F.Cu) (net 6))
 (segment (start 160.528 104.14) (end 160.528 101.346) (width 0.25) (layer F.Cu) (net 11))
 (segment (start 205.0415 106.68) (end 202.184 106.68) (width 0.25) (layer F.Cu) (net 11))
 (segment (start 205.2955 106.426) (end 205.0415 106.68) (width 0.25) (layer F.Cu) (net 11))
 (segment (start 205.2955 100.838) (end 205.2955 106.426) (width 0.25) (layer F.Cu) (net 11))
 (segment (start 204.0255 99.568) (end 205.2955 100.838) (width 0.25) (layer F.Cu) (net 11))
 (segment (start 162.306 99.568) (end 204.0255 99.568) (width 0.25) (layer F.Cu) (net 11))
 (segment (start 160.528 101.346) (end 162.306 99.568) (width 0.25) (layer F.Cu) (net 11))
 (segment (start 158.75 113.665) (end 158.75 105.918) (width 0.25) (layer F.Cu) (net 11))
 (segment (start 158.75 105.918) (end 160.528 104.14) (width 0.25) (layer F.Cu) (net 11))
 (segment (start 158.75 121.92) (end 158.75 113.665) (width 0.25) (layer F.Cu) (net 11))
 (segment (start 250.952 126.619) (end 253.0475 126.619) (width 0.25) (layer F.Cu) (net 24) (status 400000))
 (segment (start 253.111 141.478) (end 241.554 141.478) (width 0.25) (layer F.Cu) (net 24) (status 800000))
 (segment (start 253.111 126.6825) (end 253.111 141.478) (width 0.25) (layer F.Cu) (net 24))
 (segment (start 253.0475 126.619) (end 253.111 126.6825) (width 0.25) (layer F.Cu) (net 24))
 (segment (start 233.934 123.698) (end 233.299 123.698) (width 0.25) (layer F.Cu) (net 25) (status C00000))
 (segment (start 233.299 123.698) (end 232.156 122.555) (width 0.25) (layer F.Cu) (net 25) (status 400000))
 (segment (start 232.156 122.555) (end 232.156 119.5705) (width 0.25) (layer F.Cu) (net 25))
 (segment (start 232.156 119.5705) (end 234.061 117.6655) (width 0.25) (layer F.Cu) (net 25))
 (segment (start 234.061 117.6655) (end 241.6175 117.6655) (width 0.25) (layer F.Cu) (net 25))
 (segment (start 241.6175 117.6655) (end 249.4915 125.5395) (width 0.25) (layer F.Cu) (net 25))
 (segment (start 249.4915 125.5395) (end 249.4915 126.4285) (width 0.25) (layer F.Cu) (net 25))
 (segment (start 249.4915 126.4285) (end 250.952 127.889) (width 0.25) (layer F.Cu) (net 25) (status 800000))
 (segment (start 233.934 121.158) (end 233.934 119.634) (width 0.25) (layer F.Cu) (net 26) (status 400000))
 (segment (start 248.666 126.873) (end 250.952 129.159) (width 0.25) (layer F.Cu) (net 26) (status 800000))
 (segment (start 248.666 125.7935) (end 248.666 126.873) (width 0.25) (layer F.Cu) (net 26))
 (segment (start 241.8715 118.999) (end 248.666 125.7935) (width 0.25) (layer F.Cu) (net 26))
 (segment (start 234.569 118.999) (end 241.8715 118.999) (width 0.25) (layer F.Cu) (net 26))
 (segment (start 233.934 119.634) (end 234.569 118.999) (width 0.25) (layer F.Cu) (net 26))
 (segment (start 241.554 121.158) (end 241.681 121.158) (width 0.25) (layer F.Cu) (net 27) (status C00000))
 (segment (start 241.681 121.158) (end 250.952 130.429) (width 0.25) (layer F.Cu) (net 27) (status C00000))
 (segment (start 241.554 123.698) (end 242.951 123.698) (width 0.25) (layer F.Cu) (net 28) (status 400000))
 (segment (start 242.951 123.698) (end 250.952 131.699) (width 0.25) (layer F.Cu) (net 28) (status 800000))
 (segment (start 241.554 126.238) (end 244.221 126.238) (width 0.25) (layer F.Cu) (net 29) (status 400000))
 (segment (start 244.221 126.238) (end 250.952 132.969) (width 0.25) (layer F.Cu) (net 29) (status 800000))
 (segment (start 241.554 128.778) (end 245.491 128.778) (width 0.25) (layer F.Cu) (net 30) (status 400000))
 (segment (start 245.491 128.778) (end 250.952 134.239) (width 0.25) (layer F.Cu) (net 30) (status 800000))
 (segment (start 241.554 131.318) (end 246.761 131.318) (width 0.25) (layer F.Cu) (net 31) (status 400000))
 (segment (start 246.761 131.318) (end 250.952 135.509) (width 0.25) (layer F.Cu) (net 31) (status 800000))
 (segment (start 241.554 133.858) (end 248.031 133.858) (width 0.25) (layer F.Cu) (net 32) (status 400000))
 (segment (start 248.031 133.858) (end 250.952 136.779) (width 0.25) (layer F.Cu) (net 32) (status 800000)))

